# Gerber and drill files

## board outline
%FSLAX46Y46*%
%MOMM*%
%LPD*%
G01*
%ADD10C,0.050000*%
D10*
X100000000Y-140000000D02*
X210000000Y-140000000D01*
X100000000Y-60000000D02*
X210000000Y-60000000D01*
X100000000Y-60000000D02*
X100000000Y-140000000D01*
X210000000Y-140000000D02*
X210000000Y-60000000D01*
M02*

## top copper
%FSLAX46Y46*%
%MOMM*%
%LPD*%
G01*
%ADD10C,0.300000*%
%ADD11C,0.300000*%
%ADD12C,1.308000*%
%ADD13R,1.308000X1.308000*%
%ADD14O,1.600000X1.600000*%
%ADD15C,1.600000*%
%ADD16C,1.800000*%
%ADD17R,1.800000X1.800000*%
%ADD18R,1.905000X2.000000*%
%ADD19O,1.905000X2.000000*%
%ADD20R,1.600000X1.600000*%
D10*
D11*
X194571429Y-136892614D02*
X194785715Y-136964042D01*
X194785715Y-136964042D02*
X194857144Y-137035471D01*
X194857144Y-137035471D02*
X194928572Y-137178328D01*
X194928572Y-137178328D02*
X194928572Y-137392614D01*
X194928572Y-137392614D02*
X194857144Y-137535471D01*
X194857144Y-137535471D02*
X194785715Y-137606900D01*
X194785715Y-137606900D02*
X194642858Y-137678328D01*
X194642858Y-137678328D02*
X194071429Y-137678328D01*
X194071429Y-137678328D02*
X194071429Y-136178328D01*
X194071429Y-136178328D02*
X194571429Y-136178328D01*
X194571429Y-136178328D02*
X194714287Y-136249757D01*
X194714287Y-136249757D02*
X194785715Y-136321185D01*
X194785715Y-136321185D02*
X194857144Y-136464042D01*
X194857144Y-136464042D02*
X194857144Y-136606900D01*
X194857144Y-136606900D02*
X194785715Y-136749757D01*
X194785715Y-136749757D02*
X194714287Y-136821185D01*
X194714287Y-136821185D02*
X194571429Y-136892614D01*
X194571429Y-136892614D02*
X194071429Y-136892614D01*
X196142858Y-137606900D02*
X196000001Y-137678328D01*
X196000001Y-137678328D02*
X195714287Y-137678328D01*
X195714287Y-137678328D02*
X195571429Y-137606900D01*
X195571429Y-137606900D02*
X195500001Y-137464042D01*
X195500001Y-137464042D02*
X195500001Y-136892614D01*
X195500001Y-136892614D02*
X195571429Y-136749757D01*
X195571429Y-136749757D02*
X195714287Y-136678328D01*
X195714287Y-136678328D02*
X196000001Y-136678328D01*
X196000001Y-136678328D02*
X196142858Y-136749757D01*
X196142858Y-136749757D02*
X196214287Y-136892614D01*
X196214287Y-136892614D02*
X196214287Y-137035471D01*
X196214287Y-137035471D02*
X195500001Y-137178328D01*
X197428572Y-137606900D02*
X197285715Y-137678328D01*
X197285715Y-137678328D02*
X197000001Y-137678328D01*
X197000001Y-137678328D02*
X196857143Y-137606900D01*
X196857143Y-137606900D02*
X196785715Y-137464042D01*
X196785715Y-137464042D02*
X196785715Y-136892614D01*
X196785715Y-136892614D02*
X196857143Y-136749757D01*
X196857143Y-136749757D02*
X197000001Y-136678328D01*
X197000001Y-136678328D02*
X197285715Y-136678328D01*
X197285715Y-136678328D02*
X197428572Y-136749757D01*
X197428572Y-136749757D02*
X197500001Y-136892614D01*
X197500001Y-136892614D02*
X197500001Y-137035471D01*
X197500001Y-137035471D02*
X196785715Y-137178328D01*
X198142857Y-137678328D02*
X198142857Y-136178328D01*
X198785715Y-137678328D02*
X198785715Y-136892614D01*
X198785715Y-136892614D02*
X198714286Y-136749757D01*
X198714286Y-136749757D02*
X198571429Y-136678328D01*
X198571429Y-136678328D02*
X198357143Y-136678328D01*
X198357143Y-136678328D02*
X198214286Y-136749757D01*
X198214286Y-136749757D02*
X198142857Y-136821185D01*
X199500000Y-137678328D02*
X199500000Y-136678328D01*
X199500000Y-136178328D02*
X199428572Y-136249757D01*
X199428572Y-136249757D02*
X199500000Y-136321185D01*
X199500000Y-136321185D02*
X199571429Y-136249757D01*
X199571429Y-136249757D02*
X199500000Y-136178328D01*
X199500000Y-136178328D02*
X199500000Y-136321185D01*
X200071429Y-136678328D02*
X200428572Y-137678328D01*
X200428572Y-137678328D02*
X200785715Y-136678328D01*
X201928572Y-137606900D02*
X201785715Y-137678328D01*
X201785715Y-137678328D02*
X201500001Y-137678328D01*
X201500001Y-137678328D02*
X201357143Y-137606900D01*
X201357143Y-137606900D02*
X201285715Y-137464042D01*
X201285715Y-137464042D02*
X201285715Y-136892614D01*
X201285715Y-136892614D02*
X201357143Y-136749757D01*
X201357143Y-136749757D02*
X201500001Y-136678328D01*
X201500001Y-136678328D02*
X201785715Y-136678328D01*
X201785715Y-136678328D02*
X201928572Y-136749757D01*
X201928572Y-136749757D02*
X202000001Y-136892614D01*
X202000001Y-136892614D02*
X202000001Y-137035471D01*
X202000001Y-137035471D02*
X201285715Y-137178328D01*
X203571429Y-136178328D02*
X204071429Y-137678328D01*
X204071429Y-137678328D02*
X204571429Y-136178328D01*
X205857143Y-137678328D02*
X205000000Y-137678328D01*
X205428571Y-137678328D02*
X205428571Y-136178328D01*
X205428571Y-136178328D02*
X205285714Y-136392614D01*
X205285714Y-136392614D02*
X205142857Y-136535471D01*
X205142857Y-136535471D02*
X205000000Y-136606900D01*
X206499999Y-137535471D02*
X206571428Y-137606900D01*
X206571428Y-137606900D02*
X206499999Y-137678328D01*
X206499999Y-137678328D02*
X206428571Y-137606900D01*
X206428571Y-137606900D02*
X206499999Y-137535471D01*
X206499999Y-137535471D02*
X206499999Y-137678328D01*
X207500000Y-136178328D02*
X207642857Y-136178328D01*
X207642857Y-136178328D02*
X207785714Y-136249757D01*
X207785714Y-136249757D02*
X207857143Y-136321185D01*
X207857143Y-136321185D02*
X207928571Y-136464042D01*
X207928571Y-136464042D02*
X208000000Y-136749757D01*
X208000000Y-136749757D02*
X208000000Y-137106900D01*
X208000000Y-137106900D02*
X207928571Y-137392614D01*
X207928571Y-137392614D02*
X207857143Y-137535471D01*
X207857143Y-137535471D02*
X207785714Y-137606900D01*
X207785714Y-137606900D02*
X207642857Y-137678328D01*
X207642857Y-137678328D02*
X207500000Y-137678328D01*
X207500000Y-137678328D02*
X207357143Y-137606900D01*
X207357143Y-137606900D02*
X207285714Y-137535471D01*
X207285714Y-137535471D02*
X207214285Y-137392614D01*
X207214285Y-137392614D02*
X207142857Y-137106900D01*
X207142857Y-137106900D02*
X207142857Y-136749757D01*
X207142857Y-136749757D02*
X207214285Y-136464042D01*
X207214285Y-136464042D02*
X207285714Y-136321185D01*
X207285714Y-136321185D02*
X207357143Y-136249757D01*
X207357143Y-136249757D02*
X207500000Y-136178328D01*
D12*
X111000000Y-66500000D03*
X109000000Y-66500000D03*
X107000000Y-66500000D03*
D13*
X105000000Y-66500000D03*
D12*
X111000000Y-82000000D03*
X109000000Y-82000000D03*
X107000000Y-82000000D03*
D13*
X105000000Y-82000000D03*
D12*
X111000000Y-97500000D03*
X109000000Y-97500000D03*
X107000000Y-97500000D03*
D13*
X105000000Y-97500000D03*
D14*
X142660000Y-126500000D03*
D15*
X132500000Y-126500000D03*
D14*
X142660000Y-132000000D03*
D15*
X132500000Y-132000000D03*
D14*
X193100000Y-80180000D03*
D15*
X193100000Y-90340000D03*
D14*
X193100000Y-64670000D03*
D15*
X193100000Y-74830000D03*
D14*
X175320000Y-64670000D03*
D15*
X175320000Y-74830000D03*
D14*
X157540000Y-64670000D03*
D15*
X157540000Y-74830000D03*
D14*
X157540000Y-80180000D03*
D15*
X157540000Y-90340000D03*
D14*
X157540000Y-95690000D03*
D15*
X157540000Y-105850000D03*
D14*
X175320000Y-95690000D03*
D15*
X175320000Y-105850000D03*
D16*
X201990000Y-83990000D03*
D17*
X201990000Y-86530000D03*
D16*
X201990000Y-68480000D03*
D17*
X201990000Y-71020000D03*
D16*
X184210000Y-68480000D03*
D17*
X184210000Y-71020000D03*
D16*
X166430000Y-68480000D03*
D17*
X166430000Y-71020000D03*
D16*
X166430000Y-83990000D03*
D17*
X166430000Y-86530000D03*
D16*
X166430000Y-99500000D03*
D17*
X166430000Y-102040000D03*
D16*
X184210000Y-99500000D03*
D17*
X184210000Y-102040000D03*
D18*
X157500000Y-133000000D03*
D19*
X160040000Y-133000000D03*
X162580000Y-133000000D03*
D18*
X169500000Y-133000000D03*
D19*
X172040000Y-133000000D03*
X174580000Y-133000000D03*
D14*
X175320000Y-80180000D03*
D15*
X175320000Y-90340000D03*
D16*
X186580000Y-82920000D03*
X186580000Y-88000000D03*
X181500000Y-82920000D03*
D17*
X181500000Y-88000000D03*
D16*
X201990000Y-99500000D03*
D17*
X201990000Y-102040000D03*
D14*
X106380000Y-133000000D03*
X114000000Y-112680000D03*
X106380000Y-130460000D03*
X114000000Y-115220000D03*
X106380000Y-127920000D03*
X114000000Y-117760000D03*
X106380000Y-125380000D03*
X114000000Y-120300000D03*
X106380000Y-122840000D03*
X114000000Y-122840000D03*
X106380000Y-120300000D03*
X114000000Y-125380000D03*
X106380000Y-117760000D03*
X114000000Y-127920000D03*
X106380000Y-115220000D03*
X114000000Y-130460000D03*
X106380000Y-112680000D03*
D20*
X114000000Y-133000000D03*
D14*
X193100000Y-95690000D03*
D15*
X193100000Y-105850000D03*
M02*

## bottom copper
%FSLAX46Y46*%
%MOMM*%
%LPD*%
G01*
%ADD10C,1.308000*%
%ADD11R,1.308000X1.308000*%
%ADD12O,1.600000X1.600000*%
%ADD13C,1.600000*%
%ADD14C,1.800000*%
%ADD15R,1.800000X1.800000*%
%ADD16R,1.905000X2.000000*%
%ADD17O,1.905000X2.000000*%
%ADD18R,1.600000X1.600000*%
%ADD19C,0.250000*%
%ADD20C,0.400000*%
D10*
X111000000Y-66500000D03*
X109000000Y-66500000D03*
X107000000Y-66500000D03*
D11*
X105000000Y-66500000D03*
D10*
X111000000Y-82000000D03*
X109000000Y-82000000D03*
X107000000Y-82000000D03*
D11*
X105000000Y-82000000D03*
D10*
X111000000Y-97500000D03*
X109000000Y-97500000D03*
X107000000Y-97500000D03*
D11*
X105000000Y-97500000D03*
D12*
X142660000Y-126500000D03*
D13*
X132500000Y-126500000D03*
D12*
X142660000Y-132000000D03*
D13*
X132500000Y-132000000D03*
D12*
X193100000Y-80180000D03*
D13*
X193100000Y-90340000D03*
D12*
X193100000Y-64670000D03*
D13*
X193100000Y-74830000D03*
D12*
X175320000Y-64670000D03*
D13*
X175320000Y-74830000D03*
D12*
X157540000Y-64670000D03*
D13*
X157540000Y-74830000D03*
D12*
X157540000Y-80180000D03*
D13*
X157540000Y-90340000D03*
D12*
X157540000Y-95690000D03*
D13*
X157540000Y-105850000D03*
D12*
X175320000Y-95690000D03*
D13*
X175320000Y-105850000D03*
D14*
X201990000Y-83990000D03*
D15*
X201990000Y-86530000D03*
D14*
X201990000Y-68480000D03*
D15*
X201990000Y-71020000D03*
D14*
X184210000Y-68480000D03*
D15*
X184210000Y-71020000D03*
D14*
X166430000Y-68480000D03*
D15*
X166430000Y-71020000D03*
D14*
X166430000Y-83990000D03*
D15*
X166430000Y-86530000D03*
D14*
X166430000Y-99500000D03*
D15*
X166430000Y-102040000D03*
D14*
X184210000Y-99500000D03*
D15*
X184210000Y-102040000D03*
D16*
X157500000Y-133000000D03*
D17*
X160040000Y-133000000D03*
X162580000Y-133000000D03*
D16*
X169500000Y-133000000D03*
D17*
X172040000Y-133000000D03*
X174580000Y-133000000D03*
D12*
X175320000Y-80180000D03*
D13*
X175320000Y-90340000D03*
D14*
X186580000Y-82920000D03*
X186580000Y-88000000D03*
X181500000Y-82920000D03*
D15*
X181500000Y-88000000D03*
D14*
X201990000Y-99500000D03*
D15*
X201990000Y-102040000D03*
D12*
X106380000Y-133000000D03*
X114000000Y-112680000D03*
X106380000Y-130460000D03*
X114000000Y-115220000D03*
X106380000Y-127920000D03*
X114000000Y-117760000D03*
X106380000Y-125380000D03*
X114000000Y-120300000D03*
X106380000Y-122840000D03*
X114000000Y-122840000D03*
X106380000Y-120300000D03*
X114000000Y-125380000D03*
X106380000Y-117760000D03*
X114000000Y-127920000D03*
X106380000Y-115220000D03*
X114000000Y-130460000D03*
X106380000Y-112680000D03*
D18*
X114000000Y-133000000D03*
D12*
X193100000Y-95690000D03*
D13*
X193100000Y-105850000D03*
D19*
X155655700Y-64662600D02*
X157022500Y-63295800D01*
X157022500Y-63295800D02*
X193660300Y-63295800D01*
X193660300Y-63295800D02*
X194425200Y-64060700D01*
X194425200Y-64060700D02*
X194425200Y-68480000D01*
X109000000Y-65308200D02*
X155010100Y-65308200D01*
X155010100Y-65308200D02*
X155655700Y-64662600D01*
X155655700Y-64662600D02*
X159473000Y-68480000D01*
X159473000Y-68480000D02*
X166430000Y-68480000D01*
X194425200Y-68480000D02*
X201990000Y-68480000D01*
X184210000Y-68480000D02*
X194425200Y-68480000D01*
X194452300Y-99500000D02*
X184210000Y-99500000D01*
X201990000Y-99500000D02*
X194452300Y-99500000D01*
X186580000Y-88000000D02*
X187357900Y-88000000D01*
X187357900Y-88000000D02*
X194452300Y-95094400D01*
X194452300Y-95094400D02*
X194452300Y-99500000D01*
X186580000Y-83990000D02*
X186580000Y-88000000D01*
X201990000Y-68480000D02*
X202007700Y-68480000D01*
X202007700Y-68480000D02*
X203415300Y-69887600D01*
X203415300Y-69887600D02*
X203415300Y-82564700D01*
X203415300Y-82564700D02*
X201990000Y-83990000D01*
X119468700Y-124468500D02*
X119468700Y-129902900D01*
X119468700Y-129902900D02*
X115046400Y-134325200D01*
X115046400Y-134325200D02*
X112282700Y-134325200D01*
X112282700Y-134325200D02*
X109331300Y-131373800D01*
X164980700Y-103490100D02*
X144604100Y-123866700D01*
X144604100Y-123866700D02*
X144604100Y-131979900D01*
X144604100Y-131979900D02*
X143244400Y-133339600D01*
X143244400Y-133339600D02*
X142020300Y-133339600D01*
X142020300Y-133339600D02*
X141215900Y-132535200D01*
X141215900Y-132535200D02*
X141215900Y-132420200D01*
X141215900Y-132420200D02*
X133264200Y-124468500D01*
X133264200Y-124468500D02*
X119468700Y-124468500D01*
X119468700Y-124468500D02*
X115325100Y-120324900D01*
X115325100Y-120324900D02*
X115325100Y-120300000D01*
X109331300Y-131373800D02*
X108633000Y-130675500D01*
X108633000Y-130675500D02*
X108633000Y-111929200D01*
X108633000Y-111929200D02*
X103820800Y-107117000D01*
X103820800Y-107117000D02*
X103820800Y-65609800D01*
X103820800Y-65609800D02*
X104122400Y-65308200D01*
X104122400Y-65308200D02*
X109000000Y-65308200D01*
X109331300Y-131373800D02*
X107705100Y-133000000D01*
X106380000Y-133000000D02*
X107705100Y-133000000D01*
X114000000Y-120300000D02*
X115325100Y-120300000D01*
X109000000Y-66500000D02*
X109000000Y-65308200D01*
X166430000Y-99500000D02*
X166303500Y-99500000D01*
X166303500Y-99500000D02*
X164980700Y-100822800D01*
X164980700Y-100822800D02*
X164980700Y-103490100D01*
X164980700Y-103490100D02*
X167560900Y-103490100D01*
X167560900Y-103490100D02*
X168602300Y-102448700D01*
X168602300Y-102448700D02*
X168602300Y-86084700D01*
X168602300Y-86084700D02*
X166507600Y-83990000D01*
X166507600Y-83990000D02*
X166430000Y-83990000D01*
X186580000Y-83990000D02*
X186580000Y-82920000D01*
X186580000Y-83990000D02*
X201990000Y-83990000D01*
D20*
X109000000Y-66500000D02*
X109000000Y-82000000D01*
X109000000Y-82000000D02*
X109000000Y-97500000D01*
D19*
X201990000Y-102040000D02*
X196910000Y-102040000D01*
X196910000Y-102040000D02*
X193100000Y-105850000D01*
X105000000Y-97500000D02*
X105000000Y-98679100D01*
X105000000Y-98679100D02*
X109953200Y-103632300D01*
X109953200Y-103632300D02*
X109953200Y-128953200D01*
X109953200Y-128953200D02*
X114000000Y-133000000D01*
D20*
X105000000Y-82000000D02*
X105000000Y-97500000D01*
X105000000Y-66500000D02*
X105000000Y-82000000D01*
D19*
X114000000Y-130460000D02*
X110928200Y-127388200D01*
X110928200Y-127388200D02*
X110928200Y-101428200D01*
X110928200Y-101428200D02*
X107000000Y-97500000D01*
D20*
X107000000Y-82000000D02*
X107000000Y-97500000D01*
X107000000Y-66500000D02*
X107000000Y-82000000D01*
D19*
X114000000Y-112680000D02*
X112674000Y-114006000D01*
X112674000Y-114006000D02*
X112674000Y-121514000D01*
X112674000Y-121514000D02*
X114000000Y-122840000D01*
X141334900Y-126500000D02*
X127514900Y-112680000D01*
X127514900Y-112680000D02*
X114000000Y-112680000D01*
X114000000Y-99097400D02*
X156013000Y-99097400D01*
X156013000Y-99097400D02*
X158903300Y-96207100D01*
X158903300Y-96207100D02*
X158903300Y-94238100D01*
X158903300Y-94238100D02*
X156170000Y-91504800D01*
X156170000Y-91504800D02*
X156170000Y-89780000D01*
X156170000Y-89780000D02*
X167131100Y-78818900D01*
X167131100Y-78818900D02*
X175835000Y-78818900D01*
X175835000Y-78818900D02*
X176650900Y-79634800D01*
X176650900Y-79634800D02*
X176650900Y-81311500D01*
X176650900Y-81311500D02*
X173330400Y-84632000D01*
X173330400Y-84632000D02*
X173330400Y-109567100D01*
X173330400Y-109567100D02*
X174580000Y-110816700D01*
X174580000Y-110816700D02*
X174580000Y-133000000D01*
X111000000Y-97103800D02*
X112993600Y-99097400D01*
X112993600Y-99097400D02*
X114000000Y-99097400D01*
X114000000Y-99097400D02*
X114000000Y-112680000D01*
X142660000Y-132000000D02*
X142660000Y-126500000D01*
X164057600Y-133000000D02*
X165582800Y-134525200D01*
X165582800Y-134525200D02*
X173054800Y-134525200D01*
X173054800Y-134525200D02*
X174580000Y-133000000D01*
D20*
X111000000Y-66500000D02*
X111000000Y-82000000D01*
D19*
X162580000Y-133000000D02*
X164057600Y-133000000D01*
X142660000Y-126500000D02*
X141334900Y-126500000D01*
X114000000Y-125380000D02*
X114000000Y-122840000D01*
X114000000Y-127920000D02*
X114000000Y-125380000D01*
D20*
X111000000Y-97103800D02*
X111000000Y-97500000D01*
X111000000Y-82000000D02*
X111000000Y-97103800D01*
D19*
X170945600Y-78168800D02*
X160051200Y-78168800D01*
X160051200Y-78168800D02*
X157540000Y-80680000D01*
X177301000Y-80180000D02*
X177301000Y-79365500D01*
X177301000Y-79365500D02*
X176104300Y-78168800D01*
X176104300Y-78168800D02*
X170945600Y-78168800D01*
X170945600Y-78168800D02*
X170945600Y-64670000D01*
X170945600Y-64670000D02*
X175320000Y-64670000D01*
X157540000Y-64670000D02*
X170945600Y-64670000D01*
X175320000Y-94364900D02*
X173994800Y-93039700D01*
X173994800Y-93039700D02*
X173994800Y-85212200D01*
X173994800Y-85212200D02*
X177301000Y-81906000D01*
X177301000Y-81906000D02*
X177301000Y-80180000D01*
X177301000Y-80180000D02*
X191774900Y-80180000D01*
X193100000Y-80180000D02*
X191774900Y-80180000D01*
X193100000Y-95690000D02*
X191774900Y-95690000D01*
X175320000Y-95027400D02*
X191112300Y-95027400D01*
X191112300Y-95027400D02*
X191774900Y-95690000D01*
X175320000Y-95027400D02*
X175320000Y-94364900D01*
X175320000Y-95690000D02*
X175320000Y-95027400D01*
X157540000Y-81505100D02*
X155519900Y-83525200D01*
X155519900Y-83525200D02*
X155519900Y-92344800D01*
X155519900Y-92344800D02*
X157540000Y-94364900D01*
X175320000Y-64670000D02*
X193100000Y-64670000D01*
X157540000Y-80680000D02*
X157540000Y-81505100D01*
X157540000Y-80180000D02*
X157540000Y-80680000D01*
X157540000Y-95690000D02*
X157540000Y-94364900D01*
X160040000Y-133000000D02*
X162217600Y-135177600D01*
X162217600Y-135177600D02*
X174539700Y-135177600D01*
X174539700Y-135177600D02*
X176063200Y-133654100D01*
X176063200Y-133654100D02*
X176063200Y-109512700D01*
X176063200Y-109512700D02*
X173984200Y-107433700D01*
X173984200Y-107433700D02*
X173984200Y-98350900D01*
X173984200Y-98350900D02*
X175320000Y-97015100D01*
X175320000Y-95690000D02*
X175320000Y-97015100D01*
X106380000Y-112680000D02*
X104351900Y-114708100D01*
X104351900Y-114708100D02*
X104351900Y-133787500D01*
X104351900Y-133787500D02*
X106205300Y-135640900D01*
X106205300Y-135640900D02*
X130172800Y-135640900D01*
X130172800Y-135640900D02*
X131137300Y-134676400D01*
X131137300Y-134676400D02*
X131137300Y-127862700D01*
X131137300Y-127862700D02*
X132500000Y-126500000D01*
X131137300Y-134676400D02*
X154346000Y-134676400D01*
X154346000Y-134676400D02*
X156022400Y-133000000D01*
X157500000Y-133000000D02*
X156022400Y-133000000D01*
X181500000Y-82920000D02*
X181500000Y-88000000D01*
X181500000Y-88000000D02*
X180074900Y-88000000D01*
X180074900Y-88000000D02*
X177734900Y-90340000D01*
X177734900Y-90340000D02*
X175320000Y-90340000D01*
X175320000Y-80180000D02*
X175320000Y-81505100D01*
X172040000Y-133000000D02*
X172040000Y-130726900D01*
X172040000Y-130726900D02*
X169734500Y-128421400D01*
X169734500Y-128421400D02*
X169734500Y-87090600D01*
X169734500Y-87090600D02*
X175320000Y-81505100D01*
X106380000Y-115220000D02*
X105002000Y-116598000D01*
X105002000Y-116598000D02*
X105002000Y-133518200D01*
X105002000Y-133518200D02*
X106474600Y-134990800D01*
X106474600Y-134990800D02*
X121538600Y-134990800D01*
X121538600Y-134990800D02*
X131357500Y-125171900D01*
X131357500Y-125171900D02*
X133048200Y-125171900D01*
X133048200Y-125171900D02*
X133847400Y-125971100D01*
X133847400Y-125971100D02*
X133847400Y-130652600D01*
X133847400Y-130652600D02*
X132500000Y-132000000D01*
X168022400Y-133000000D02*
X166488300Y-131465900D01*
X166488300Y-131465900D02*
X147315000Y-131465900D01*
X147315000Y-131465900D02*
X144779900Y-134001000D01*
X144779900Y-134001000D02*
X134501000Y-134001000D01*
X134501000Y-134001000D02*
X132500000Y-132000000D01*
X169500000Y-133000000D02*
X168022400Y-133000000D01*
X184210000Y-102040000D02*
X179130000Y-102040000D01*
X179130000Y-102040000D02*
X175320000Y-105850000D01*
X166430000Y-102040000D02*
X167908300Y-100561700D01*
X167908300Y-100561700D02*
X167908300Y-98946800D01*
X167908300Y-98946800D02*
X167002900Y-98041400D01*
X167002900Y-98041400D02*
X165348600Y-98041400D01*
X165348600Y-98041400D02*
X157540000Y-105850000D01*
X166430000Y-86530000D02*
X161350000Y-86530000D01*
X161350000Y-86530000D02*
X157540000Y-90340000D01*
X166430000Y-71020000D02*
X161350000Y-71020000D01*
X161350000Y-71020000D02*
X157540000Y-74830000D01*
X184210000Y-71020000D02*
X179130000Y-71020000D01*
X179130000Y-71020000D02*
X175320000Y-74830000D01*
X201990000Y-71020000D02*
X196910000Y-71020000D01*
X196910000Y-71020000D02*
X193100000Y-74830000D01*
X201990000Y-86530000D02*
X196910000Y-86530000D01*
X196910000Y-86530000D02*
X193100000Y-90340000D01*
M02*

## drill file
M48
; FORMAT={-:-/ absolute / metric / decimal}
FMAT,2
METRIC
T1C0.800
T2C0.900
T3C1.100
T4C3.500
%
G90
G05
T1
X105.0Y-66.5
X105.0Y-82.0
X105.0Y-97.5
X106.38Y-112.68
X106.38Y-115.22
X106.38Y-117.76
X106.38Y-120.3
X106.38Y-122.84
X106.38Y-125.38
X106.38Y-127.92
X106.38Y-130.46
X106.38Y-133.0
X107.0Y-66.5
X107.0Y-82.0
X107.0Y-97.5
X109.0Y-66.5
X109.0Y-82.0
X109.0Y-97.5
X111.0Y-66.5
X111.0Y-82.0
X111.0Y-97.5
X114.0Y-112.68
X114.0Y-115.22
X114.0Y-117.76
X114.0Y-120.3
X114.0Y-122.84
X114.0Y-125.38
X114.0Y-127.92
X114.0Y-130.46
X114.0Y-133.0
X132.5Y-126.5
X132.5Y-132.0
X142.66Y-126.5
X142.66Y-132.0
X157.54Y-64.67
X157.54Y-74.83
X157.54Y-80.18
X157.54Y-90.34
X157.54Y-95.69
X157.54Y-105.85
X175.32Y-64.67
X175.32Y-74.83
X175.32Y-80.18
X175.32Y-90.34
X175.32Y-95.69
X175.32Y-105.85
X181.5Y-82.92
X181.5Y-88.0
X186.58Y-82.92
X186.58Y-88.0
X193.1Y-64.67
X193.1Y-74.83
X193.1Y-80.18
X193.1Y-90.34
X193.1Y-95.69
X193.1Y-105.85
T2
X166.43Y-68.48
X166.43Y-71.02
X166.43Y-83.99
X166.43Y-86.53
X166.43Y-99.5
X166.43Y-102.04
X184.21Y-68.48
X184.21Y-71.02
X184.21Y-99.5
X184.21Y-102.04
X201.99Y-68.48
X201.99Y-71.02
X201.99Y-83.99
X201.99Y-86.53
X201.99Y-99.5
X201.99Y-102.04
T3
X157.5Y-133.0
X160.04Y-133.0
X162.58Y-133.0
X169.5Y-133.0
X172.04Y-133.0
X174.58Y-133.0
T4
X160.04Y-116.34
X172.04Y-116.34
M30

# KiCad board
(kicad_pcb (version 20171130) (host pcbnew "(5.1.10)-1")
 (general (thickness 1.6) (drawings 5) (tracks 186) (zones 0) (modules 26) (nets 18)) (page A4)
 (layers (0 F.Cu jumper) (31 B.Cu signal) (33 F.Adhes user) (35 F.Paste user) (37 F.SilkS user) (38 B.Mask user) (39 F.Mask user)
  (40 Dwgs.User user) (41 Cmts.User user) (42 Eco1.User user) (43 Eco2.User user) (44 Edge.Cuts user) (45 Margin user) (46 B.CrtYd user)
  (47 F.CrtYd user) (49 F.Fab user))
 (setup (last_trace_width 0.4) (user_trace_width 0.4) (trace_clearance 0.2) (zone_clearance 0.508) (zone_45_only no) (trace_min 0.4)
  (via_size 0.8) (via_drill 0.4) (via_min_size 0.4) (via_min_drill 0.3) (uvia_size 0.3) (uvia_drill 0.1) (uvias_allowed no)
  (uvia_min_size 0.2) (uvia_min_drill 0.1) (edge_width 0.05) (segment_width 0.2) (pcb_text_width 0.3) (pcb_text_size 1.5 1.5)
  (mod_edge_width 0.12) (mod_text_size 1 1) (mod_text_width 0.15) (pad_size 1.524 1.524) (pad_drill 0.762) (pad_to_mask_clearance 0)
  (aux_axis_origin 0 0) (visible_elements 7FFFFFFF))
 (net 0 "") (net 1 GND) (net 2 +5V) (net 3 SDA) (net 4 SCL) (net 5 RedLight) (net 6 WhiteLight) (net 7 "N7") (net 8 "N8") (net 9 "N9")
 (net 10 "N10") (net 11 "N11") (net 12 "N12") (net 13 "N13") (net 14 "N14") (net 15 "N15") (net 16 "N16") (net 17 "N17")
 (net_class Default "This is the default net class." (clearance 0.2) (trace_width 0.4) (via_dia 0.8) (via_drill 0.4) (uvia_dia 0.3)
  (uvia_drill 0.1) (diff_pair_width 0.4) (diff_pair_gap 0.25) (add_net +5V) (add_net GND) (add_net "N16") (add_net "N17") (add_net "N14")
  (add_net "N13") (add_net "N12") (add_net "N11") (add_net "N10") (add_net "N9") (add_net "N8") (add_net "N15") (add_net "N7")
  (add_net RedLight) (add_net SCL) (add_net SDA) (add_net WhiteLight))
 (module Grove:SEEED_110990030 (layer F.Cu) (at 108 66.5)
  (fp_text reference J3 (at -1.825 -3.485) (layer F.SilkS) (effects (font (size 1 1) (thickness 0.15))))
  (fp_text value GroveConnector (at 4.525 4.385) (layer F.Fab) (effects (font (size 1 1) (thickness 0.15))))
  (pad 4 thru_hole circle (at 3 0) (size 1.308 1.308) (drill 0.8) (layers *.Cu *.Mask) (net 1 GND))
  (pad 3 thru_hole circle (at 1 0) (size 1.308 1.308) (drill 0.8) (layers *.Cu *.Mask) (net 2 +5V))
  (pad 2 thru_hole circle (at -1 0) (size 1.308 1.308) (drill 0.8) (layers *.Cu *.Mask) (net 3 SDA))
  (pad 1 thru_hole rect (at -3 0) (size 1.308 1.308) (drill 0.8) (layers *.Cu *.Mask) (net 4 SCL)))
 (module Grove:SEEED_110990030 (layer F.Cu) (at 108 82)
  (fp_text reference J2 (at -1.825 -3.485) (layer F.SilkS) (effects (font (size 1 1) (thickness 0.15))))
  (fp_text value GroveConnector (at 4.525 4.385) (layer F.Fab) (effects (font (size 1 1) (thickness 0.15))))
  (pad 4 thru_hole circle (at 3 0) (size 1.308 1.308) (drill 0.8) (layers *.Cu *.Mask) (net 1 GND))
  (pad 3 thru_hole circle (at 1 0) (size 1.308 1.308) (drill 0.8) (layers *.Cu *.Mask) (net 2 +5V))
  (pad 2 thru_hole circle (at -1 0) (size 1.308 1.308) (drill 0.8) (layers *.Cu *.Mask) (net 3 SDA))
  (pad 1 thru_hole rect (at -3 0) (size 1.308 1.308) (drill 0.8) (layers *.Cu *.Mask) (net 4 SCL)))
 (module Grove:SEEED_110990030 (layer F.Cu) (at 108 97.5)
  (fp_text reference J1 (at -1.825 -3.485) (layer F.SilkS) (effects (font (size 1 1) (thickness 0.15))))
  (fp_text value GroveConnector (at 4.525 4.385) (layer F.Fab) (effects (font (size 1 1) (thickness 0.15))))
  (pad 4 thru_hole circle (at 3 0) (size 1.308 1.308) (drill 0.8) (layers *.Cu *.Mask) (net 1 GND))
  (pad 3 thru_hole circle (at 1 0) (size 1.308 1.308) (drill 0.8) (layers *.Cu *.Mask) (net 2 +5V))
  (pad 2 thru_hole circle (at -1 0) (size 1.308 1.308) (drill 0.8) (layers *.Cu *.Mask) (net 3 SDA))
  (pad 1 thru_hole rect (at -3 0) (size 1.308 1.308) (drill 0.8) (layers *.Cu *.Mask) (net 4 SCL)))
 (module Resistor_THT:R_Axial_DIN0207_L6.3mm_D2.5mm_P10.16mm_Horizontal (layer F.Cu) (at 132.5 126.5)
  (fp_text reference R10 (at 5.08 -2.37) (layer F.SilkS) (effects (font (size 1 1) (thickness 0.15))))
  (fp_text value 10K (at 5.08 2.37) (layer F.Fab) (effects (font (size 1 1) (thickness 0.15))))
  (pad 2 thru_hole oval (at 10.16 0) (size 1.6 1.6) (drill 0.8) (layers *.Cu *.Mask) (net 1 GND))
  (pad 1 thru_hole circle (at 0 0) (size 1.6 1.6) (drill 0.8) (layers *.Cu *.Mask) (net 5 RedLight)))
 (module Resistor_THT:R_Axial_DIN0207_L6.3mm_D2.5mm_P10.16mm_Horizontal (layer F.Cu) (at 132.5 132)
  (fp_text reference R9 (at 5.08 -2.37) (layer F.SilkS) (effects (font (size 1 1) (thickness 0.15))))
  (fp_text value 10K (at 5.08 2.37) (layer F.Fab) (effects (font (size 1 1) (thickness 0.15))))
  (pad 2 thru_hole oval (at 10.16 0) (size 1.6 1.6) (drill 0.8) (layers *.Cu *.Mask) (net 1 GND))
  (pad 1 thru_hole circle (at 0 0) (size 1.6 1.6) (drill 0.8) (layers *.Cu *.Mask) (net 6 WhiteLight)))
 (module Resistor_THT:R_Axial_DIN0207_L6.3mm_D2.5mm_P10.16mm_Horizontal (layer F.Cu) (at 193.1 90.34 90)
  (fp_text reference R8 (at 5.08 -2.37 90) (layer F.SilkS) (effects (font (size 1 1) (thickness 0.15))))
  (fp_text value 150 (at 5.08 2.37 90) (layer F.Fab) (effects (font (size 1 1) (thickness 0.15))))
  (pad 2 thru_hole oval (at 10.16 0 90) (size 1.6 1.6) (drill 0.8) (layers *.Cu *.Mask) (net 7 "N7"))
  (pad 1 thru_hole circle (at 0 0 90) (size 1.6 1.6) (drill 0.8) (layers *.Cu *.Mask) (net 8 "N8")))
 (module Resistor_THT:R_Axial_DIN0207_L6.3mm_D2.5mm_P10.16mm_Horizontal (layer F.Cu) (at 193.1 74.83 90)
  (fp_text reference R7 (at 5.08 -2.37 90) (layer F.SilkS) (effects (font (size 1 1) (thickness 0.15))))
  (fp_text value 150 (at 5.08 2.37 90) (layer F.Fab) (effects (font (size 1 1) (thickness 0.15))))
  (pad 2 thru_hole oval (at 10.16 0 90) (size 1.6 1.6) (drill 0.8) (layers *.Cu *.Mask) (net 7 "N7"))
  (pad 1 thru_hole circle (at 0 0 90) (size 1.6 1.6) (drill 0.8) (layers *.Cu *.Mask) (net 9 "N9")))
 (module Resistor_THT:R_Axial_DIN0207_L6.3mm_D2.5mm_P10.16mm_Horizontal (layer F.Cu) (at 175.32 74.83 90)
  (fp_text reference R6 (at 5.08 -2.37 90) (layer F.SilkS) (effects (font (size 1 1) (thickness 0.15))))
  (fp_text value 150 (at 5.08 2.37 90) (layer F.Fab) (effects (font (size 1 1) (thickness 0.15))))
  (pad 2 thru_hole oval (at 10.16 0 90) (size 1.6 1.6) (drill 0.8) (layers *.Cu *.Mask) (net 7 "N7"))
  (pad 1 thru_hole circle (at 0 0 90) (size 1.6 1.6) (drill 0.8) (layers *.Cu *.Mask) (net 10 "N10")))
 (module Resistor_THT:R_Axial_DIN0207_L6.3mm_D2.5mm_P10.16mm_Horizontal (layer F.Cu) (at 157.54 74.83 90)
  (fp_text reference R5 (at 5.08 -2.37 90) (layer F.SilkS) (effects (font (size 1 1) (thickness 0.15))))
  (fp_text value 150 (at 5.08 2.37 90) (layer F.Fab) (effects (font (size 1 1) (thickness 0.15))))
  (pad 2 thru_hole oval (at 10.16 0 90) (size 1.6 1.6) (drill 0.8) (layers *.Cu *.Mask) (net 7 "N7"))
  (pad 1 thru_hole circle (at 0 0 90) (size 1.6 1.6) (drill 0.8) (layers *.Cu *.Mask) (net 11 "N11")))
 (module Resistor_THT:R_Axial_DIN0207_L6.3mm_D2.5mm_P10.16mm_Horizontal (layer F.Cu) (at 157.54 90.34 90)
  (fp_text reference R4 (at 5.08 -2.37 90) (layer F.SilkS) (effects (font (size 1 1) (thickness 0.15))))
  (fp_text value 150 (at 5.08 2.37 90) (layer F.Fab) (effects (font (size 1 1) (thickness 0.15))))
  (pad 2 thru_hole oval (at 10.16 0 90) (size 1.6 1.6) (drill 0.8) (layers *.Cu *.Mask) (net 7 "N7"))
  (pad 1 thru_hole circle (at 0 0 90) (size 1.6 1.6) (drill 0.8) (layers *.Cu *.Mask) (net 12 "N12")))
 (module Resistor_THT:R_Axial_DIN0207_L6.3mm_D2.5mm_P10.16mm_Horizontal (layer F.Cu) (at 157.54 105.85 90)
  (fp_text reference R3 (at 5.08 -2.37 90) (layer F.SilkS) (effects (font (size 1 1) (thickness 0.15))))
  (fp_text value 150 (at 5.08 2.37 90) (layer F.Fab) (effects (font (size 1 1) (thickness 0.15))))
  (pad 2 thru_hole oval (at 10.16 0 90) (size 1.6 1.6) (drill 0.8) (layers *.Cu *.Mask) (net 7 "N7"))
  (pad 1 thru_hole circle (at 0 0 90) (size 1.6 1.6) (drill 0.8) (layers *.Cu *.Mask) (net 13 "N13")))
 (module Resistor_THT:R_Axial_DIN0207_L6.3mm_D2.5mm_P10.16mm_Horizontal (layer F.Cu) (at 175.32 105.85 90)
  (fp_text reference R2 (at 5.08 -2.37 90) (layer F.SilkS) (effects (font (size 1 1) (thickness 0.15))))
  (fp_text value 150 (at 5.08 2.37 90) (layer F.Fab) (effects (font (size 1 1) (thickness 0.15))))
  (pad 2 thru_hole oval (at 10.16 0 90) (size 1.6 1.6) (drill 0.8) (layers *.Cu *.Mask) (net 7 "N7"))
  (pad 1 thru_hole circle (at 0 0 90) (size 1.6 1.6) (drill 0.8) (layers *.Cu *.Mask) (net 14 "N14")))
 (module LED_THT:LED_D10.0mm (layer F.Cu) (at 201.99 86.53 90)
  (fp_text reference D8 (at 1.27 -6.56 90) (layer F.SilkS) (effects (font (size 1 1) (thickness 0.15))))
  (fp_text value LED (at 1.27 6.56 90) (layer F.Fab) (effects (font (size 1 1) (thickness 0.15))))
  (pad 2 thru_hole circle (at 2.54 0 90) (size 1.8 1.8) (drill 0.9) (layers *.Cu *.Mask) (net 2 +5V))
  (pad 1 thru_hole rect (at 0 0 90) (size 1.8 1.8) (drill 0.9) (layers *.Cu *.Mask) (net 8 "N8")))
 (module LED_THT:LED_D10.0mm (layer F.Cu) (at 201.99 71.02 90)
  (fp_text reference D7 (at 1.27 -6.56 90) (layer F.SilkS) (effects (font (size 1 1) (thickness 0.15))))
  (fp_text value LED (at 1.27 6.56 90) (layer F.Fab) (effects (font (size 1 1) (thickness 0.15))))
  (pad 2 thru_hole circle (at 2.54 0 90) (size 1.8 1.8) (drill 0.9) (layers *.Cu *.Mask) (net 2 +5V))
  (pad 1 thru_hole rect (at 0 0 90) (size 1.8 1.8) (drill 0.9) (layers *.Cu *.Mask) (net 9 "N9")))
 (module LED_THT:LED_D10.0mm (layer F.Cu) (at 184.21 71.02 90)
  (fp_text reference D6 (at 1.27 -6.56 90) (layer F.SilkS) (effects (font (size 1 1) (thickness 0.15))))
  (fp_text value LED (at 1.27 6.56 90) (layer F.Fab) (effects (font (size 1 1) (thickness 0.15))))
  (pad 2 thru_hole circle (at 2.54 0 90) (size 1.8 1.8) (drill 0.9) (layers *.Cu *.Mask) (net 2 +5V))
  (pad 1 thru_hole rect (at 0 0 90) (size 1.8 1.8) (drill 0.9) (layers *.Cu *.Mask) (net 10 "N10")))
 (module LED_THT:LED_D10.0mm (layer F.Cu) (at 166.43 71.02 90)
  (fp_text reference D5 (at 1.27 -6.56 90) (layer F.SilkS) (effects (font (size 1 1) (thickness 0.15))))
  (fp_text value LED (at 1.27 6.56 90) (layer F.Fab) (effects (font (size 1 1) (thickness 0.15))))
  (pad 2 thru_hole circle (at 2.54 0 90) (size 1.8 1.8) (drill 0.9) (layers *.Cu *.Mask) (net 2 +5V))
  (pad 1 thru_hole rect (at 0 0 90) (size 1.8 1.8) (drill 0.9) (layers *.Cu *.Mask) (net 11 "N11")))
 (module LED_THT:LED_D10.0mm (layer F.Cu) (at 166.43 86.53 90)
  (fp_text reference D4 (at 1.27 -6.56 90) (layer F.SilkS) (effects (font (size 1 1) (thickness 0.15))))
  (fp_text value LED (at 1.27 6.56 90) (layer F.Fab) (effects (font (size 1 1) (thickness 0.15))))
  (pad 2 thru_hole circle (at 2.54 0 90) (size 1.8 1.8) (drill 0.9) (layers *.Cu *.Mask) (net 2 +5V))
  (pad 1 thru_hole rect (at 0 0 90) (size 1.8 1.8) (drill 0.9) (layers *.Cu *.Mask) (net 12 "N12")))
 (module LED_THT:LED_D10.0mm (layer F.Cu) (at 166.43 102.04 90)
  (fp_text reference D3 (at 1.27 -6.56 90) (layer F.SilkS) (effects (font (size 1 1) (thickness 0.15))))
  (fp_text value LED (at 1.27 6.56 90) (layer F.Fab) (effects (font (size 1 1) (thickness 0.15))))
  (pad 2 thru_hole circle (at 2.54 0 90) (size 1.8 1.8) (drill 0.9) (layers *.Cu *.Mask) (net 2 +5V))
  (pad 1 thru_hole rect (at 0 0 90) (size 1.8 1.8) (drill 0.9) (layers *.Cu *.Mask) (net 13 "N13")))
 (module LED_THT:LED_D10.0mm (layer F.Cu) (at 184.21 102.04 90)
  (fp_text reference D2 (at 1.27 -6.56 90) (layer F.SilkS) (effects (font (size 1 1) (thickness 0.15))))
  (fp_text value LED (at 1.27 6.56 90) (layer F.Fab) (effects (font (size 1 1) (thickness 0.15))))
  (pad 2 thru_hole circle (at 2.54 0 90) (size 1.8 1.8) (drill 0.9) (layers *.Cu *.Mask) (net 2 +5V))
  (pad 1 thru_hole rect (at 0 0 90) (size 1.8 1.8) (drill 0.9) (layers *.Cu *.Mask) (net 14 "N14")))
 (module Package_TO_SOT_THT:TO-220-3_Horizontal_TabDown (layer F.Cu) (at 157.5 133)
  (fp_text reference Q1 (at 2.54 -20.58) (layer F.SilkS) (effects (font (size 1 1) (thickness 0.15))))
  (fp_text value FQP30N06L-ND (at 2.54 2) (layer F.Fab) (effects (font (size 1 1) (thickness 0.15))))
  (pad "" np_thru_hole oval (at 2.54 -16.66) (size 3.5 3.5) (drill 3.5) (layers *.Cu *.Mask))
  (pad 1 thru_hole rect (at 0 0) (size 1.905 2) (drill 1.1) (layers *.Cu *.Mask) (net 5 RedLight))
  (pad 2 thru_hole oval (at 2.54 0) (size 1.905 2) (drill 1.1) (layers *.Cu *.Mask) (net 7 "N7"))
  (pad 3 thru_hole oval (at 5.08 0) (size 1.905 2) (drill 1.1) (layers *.Cu *.Mask) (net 1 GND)))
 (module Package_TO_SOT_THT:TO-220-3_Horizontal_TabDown (layer F.Cu) (at 169.5 133)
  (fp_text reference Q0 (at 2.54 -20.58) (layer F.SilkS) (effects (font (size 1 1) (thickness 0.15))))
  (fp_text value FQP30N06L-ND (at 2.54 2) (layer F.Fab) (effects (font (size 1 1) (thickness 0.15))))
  (pad "" np_thru_hole oval (at 2.54 -16.66) (size 3.5 3.5) (drill 3.5) (layers *.Cu *.Mask))
  (pad 1 thru_hole rect (at 0 0) (size 1.905 2) (drill 1.1) (layers *.Cu *.Mask) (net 6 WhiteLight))
  (pad 2 thru_hole oval (at 2.54 0) (size 1.905 2) (drill 1.1) (layers *.Cu *.Mask) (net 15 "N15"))
  (pad 3 thru_hole oval (at 5.08 0) (size 1.905 2) (drill 1.1) (layers *.Cu *.Mask) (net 1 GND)))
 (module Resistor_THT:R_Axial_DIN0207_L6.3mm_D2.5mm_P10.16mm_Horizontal (layer F.Cu) (at 175.32 90.34 90)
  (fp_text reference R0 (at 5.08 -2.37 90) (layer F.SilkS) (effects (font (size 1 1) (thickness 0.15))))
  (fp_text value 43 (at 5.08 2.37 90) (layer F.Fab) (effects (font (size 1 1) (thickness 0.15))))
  (pad 2 thru_hole oval (at 10.16 0 90) (size 1.6 1.6) (drill 0.8) (layers *.Cu *.Mask) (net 15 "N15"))
  (pad 1 thru_hole circle (at 0 0 90) (size 1.6 1.6) (drill 0.8) (layers *.Cu *.Mask) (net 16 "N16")))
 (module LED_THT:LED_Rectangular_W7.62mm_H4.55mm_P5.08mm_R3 (layer F.Cu) (at 181.5 88 90)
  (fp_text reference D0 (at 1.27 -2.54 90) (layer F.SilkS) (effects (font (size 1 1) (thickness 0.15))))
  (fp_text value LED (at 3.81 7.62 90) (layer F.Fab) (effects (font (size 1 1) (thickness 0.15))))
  (pad 2 thru_hole circle (at 5.08 5.08 90) (size 1.8 1.8) (drill 0.8) (layers *.Cu *.Mask) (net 2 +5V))
  (pad 2 thru_hole circle (at 0 5.08 90) (size 1.8 1.8) (drill 0.8) (layers *.Cu *.Mask) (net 2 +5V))
  (pad 1 thru_hole circle (at 5.08 0 90) (size 1.8 1.8) (drill 0.8) (layers *.Cu *.Mask) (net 16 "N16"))
  (pad 1 thru_hole rect (at 0 0 90) (size 1.8 1.8) (drill 0.8) (layers *.Cu *.Mask) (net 16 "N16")))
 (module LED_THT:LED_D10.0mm (layer F.Cu) (at 201.99 102.04 90)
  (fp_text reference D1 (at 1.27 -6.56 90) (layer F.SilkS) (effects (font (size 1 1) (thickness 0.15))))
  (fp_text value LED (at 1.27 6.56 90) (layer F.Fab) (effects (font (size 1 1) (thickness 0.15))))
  (pad 2 thru_hole circle (at 2.54 0 90) (size 1.8 1.8) (drill 0.9) (layers *.Cu *.Mask) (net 2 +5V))
  (pad 1 thru_hole rect (at 0 0 90) (size 1.8 1.8) (drill 0.9) (layers *.Cu *.Mask) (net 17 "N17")))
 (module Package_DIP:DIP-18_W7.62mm (layer F.Cu) (at 114 133 180)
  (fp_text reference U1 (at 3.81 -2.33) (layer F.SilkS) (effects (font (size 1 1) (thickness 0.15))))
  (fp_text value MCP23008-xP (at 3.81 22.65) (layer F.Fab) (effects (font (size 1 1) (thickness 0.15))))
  (pad 18 thru_hole oval (at 7.62 0 180) (size 1.6 1.6) (drill 0.8) (layers *.Cu *.Mask) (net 2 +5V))
  (pad 9 thru_hole oval (at 0 20.32 180) (size 1.6 1.6) (drill 0.8) (layers *.Cu *.Mask) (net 1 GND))
  (pad 17 thru_hole oval (at 7.62 2.54 180) (size 1.6 1.6) (drill 0.8) (layers *.Cu *.Mask))
  (pad 8 thru_hole oval (at 0 17.78 180) (size 1.6 1.6) (drill 0.8) (layers *.Cu *.Mask))
  (pad 16 thru_hole oval (at 7.62 5.08 180) (size 1.6 1.6) (drill 0.8) (layers *.Cu *.Mask))
  (pad 7 thru_hole oval (at 0 15.24 180) (size 1.6 1.6) (drill 0.8) (layers *.Cu *.Mask))
  (pad 15 thru_hole oval (at 7.62 7.62 180) (size 1.6 1.6) (drill 0.8) (layers *.Cu *.Mask))
  (pad 6 thru_hole oval (at 0 12.7 180) (size 1.6 1.6) (drill 0.8) (layers *.Cu *.Mask) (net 2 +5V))
  (pad 14 thru_hole oval (at 7.62 10.16 180) (size 1.6 1.6) (drill 0.8) (layers *.Cu *.Mask))
  (pad 5 thru_hole oval (at 0 10.16 180) (size 1.6 1.6) (drill 0.8) (layers *.Cu *.Mask) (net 1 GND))
  (pad 13 thru_hole oval (at 7.62 12.7 180) (size 1.6 1.6) (drill 0.8) (layers *.Cu *.Mask))
  (pad 4 thru_hole oval (at 0 7.62 180) (size 1.6 1.6) (drill 0.8) (layers *.Cu *.Mask) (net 1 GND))
  (pad 12 thru_hole oval (at 7.62 15.24 180) (size 1.6 1.6) (drill 0.8) (layers *.Cu *.Mask))
  (pad 3 thru_hole oval (at 0 5.08 180) (size 1.6 1.6) (drill 0.8) (layers *.Cu *.Mask) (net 1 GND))
  (pad 11 thru_hole oval (at 7.62 17.78 180) (size 1.6 1.6) (drill 0.8) (layers *.Cu *.Mask) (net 6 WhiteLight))
  (pad 2 thru_hole oval (at 0 2.54 180) (size 1.6 1.6) (drill 0.8) (layers *.Cu *.Mask) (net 3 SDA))
  (pad 10 thru_hole oval (at 7.62 20.32 180) (size 1.6 1.6) (drill 0.8) (layers *.Cu *.Mask) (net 5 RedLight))
  (pad 1 thru_hole rect (at 0 0 180) (size 1.6 1.6) (drill 0.8) (layers *.Cu *.Mask) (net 4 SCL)))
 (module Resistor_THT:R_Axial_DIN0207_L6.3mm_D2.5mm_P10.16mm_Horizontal (layer F.Cu) (at 193.1 105.85 90)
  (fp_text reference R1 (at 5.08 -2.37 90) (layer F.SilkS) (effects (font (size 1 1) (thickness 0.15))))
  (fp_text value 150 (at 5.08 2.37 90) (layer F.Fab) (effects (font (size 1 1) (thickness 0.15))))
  (pad 2 thru_hole oval (at 10.16 0 90) (size 1.6 1.6) (drill 0.8) (layers *.Cu *.Mask) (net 7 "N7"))
  (pad 1 thru_hole circle (at 0 0 90) (size 1.6 1.6) (drill 0.8) (layers *.Cu *.Mask) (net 17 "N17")))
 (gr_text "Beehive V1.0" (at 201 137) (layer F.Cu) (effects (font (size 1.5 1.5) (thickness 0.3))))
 (gr_line (start 100 140) (end 210 140) (layer Edge.Cuts) (width 0.05))
 (gr_line (start 100 60) (end 210 60) (layer Edge.Cuts) (width 0.05))
 (gr_line (start 100 60) (end 100 140) (layer Edge.Cuts) (width 0.05))
 (gr_line (start 210 140) (end 210 60) (layer Edge.Cuts) (width 0.05))
 (segment (start 155.6557 64.6626) (end 157.0225 63.2958) (width 0.25) (layer B.Cu) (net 2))
 (segment (start 157.0225 63.2958) (end 193.6603 63.2958) (width 0.25) (layer B.Cu) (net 2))
 (segment (start 193.6603 63.2958) (end 194.4252 64.0607) (width 0.25) (layer B.Cu) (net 2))
 (segment (start 194.4252 64.0607) (end 194.4252 68.48) (width 0.25) (layer B.Cu) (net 2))
 (segment (start 109 65.3082) (end 155.0101 65.3082) (width 0.25) (layer B.Cu) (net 2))
 (segment (start 155.0101 65.3082) (end 155.6557 64.6626) (width 0.25) (layer B.Cu) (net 2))
 (segment (start 155.6557 64.6626) (end 159.473 68.48) (width 0.25) (layer B.Cu) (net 2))
 (segment (start 159.473 68.48) (end 166.43 68.48) (width 0.25) (layer B.Cu) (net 2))
 (segment (start 194.4252 68.48) (end 201.99 68.48) (width 0.25) (layer B.Cu) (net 2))
 (segment (start 184.21 68.48) (end 194.4252 68.48) (width 0.25) (layer B.Cu) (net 2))
 (segment (start 194.4523 99.5) (end 184.21 99.5) (width 0.25) (layer B.Cu) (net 2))
 (segment (start 201.99 99.5) (end 194.4523 99.5) (width 0.25) (layer B.Cu) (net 2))
 (segment (start 186.58 88) (end 187.3579 88) (width 0.25) (layer B.Cu) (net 2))
 (segment (start 187.3579 88) (end 194.4523 95.0944) (width 0.25) (layer B.Cu) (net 2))
 (segment (start 194.4523 95.0944) (end 194.4523 99.5) (width 0.25) (layer B.Cu) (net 2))
 (segment (start 186.58 83.99) (end 186.58 88) (width 0.25) (layer B.Cu) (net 2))
 (segment (start 201.99 68.48) (end 202.0077 68.48) (width 0.25) (layer B.Cu) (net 2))
 (segment (start 202.0077 68.48) (end 203.4153 69.8876) (width 0.25) (layer B.Cu) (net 2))
 (segment (start 203.4153 69.8876) (end 203.4153 82.5647) (width 0.25) (layer B.Cu) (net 2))
 (segment (start 203.4153 82.5647) (end 201.99 83.99) (width 0.25) (layer B.Cu) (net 2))
 (segment (start 119.4687 124.4685) (end 119.4687 129.9029) (width 0.25) (layer B.Cu) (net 2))
 (segment (start 119.4687 129.9029) (end 115.0464 134.3252) (width 0.25) (layer B.Cu) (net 2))
 (segment (start 115.0464 134.3252) (end 112.2827 134.3252) (width 0.25) (layer B.Cu) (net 2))
 (segment (start 112.2827 134.3252) (end 109.3313 131.3738) (width 0.25) (layer B.Cu) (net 2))
 (segment (start 164.9807 103.4901) (end 144.6041 123.8667) (width 0.25) (layer B.Cu) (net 2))
 (segment (start 144.6041 123.8667) (end 144.6041 131.9799) (width 0.25) (layer B.Cu) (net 2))
 (segment (start 144.6041 131.9799) (end 143.2444 133.3396) (width 0.25) (layer B.Cu) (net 2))
 (segment (start 143.2444 133.3396) (end 142.0203 133.3396) (width 0.25) (layer B.Cu) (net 2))
 (segment (start 142.0203 133.3396) (end 141.2159 132.5352) (width 0.25) (layer B.Cu) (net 2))
 (segment (start 141.2159 132.5352) (end 141.2159 132.4202) (width 0.25) (layer B.Cu) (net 2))
 (segment (start 141.2159 132.4202) (end 133.2642 124.4685) (width 0.25) (layer B.Cu) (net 2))
 (segment (start 133.2642 124.4685) (end 119.4687 124.4685) (width 0.25) (layer B.Cu) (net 2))
 (segment (start 119.4687 124.4685) (end 115.3251 120.3249) (width 0.25) (layer B.Cu) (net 2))
 (segment (start 115.3251 120.3249) (end 115.3251 120.3) (width 0.25) (layer B.Cu) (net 2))
 (segment (start 109.3313 131.3738) (end 108.633 130.6755) (width 0.25) (layer B.Cu) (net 2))
 (segment (start 108.633 130.6755) (end 108.633 111.9292) (width 0.25) (layer B.Cu) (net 2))
 (segment (start 108.633 111.9292) (end 103.8208 107.117) (width 0.25) (layer B.Cu) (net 2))
 (segment (start 103.8208 107.117) (end 103.8208 65.6098) (width 0.25) (layer B.Cu) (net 2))
 (segment (start 103.8208 65.6098) (end 104.1224 65.3082) (width 0.25) (layer B.Cu) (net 2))
 (segment (start 104.1224 65.3082) (end 109 65.3082) (width 0.25) (layer B.Cu) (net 2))
 (segment (start 109.3313 131.3738) (end 107.7051 133) (width 0.25) (layer B.Cu) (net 2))
 (segment (start 106.38 133) (end 107.7051 133) (width 0.25) (layer B.Cu) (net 2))
 (segment (start 114 120.3) (end 115.3251 120.3) (width 0.25) (layer B.Cu) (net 2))
 (segment (start 109 66.5) (end 109 65.3082) (width 0.25) (layer B.Cu) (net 2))
 (segment (start 166.43 99.5) (end 166.3035 99.5) (width 0.25) (layer B.Cu) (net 2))
 (segment (start 166.3035 99.5) (end 164.9807 100.8228) (width 0.25) (layer B.Cu) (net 2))
 (segment (start 164.9807 100.8228) (end 164.9807 103.4901) (width 0.25) (layer B.Cu) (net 2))
 (segment (start 164.9807 103.4901) (end 167.5609 103.4901) (width 0.25) (layer B.Cu) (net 2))
 (segment (start 167.5609 103.4901) (end 168.6023 102.4487) (width 0.25) (layer B.Cu) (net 2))
 (segment (start 168.6023 102.4487) (end 168.6023 86.0847) (width 0.25) (layer B.Cu) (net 2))
 (segment (start 168.6023 86.0847) (end 166.5076 83.99) (width 0.25) (layer B.Cu) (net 2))
 (segment (start 166.5076 83.99) (end 166.43 83.99) (width 0.25) (layer B.Cu) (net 2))
 (segment (start 186.58 83.99) (end 186.58 82.92) (width 0.25) (layer B.Cu) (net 2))
 (segment (start 186.58 83.99) (end 201.99 83.99) (width 0.25) (layer B.Cu) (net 2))
 (segment (start 109 66.5) (end 109 82) (width 0.4) (layer B.Cu) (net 2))
 (segment (start 109 82) (end 109 97.5) (width 0.4) (layer B.Cu) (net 2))
 (segment (start 201.99 102.04) (end 196.91 102.04) (width 0.25) (layer B.Cu) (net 17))
 (segment (start 196.91 102.04) (end 193.1 105.85) (width 0.25) (layer B.Cu) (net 17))
 (segment (start 105 97.5) (end 105 98.6791) (width 0.25) (layer B.Cu) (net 4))
 (segment (start 105 98.6791) (end 109.9532 103.6323) (width 0.25) (layer B.Cu) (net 4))
 (segment (start 109.9532 103.6323) (end 109.9532 128.9532) (width 0.25) (layer B.Cu) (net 4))
 (segment (start 109.9532 128.9532) (end 114 133) (width 0.25) (layer B.Cu) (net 4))
 (segment (start 105 82) (end 105 97.5) (width 0.4) (layer B.Cu) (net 4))
 (segment (start 105 66.5) (end 105 82) (width 0.4) (layer B.Cu) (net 4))
 (segment (start 114 130.46) (end 110.9282 127.3882) (width 0.25) (layer B.Cu) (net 3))
 (segment (start 110.9282 127.3882) (end 110.9282 101.4282) (width 0.25) (layer B.Cu) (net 3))
 (segment (start 110.9282 101.4282) (end 107 97.5) (width 0.25) (layer B.Cu) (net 3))
 (segment (start 107 82) (end 107 97.5) (width 0.4) (layer B.Cu) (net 3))
 (segment (start 107 66.5) (end 107 82) (width 0.4) (layer B.Cu) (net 3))
 (segment (start 114 112.68) (end 112.674 114.006) (width 0.25) (layer B.Cu) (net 1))
 (segment (start 112.674 114.006) (end 112.674 121.514) (width 0.25) (layer B.Cu) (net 1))
 (segment (start 112.674 121.514) (end 114 122.84) (width 0.25) (layer B.Cu) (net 1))
 (segment (start 141.3349 126.5) (end 127.5149 112.68) (width 0.25) (layer B.Cu) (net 1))
 (segment (start 127.5149 112.68) (end 114 112.68) (width 0.25) (layer B.Cu) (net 1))
 (segment (start 114 99.0974) (end 156.013 99.0974) (width 0.25) (layer B.Cu) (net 1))
 (segment (start 156.013 99.0974) (end 158.9033 96.2071) (width 0.25) (layer B.Cu) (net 1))
 (segment (start 158.9033 96.2071) (end 158.9033 94.2381) (width 0.25) (layer B.Cu) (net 1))
 (segment (start 158.9033 94.2381) (end 156.17 91.5048) (width 0.25) (layer B.Cu) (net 1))
 (segment (start 156.17 91.5048) (end 156.17 89.78) (width 0.25) (layer B.Cu) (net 1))
 (segment (start 156.17 89.78) (end 167.1311 78.8189) (width 0.25) (layer B.Cu) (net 1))
 (segment (start 167.1311 78.8189) (end 175.835 78.8189) (width 0.25) (layer B.Cu) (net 1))
 (segment (start 175.835 78.8189) (end 176.6509 79.6348) (width 0.25) (layer B.Cu) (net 1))
 (segment (start 176.6509 79.6348) (end 176.6509 81.3115) (width 0.25) (layer B.Cu) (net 1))
 (segment (start 176.6509 81.3115) (end 173.3304 84.632) (width 0.25) (layer B.Cu) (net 1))
 (segment (start 173.3304 84.632) (end 173.3304 109.5671) (width 0.25) (layer B.Cu) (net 1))
 (segment (start 173.3304 109.5671) (end 174.58 110.8167) (width 0.25) (layer B.Cu) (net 1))
 (segment (start 174.58 110.8167) (end 174.58 133) (width 0.25) (layer B.Cu) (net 1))
 (segment (start 111 97.1038) (end 112.9936 99.0974) (width 0.25) (layer B.Cu) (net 1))
 (segment (start 112.9936 99.0974) (end 114 99.0974) (width 0.25) (layer B.Cu) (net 1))
 (segment (start 114 99.0974) (end 114 112.68) (width 0.25) (layer B.Cu) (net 1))
 (segment (start 142.66 132) (end 142.66 126.5) (width 0.25) (layer B.Cu) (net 1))
 (segment (start 164.0576 133) (end 165.5828 134.5252) (width 0.25) (layer B.Cu) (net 1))
 (segment (start 165.5828 134.5252) (end 173.0548 134.5252) (width 0.25) (layer B.Cu) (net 1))
 (segment (start 173.0548 134.5252) (end 174.58 133) (width 0.25) (layer B.Cu) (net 1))
 (segment (start 111 66.5) (end 111 82) (width 0.4) (layer B.Cu) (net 1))
 (segment (start 162.58 133) (end 164.0576 133) (width 0.25) (layer B.Cu) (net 1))
 (segment (start 142.66 126.5) (end 141.3349 126.5) (width 0.25) (layer B.Cu) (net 1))
 (segment (start 114 125.38) (end 114 122.84) (width 0.25) (layer B.Cu) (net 1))
 (segment (start 114 127.92) (end 114 125.38) (width 0.25) (layer B.Cu) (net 1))
 (segment (start 111 97.1038) (end 111 97.5) (width 0.4) (layer B.Cu) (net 1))
 (segment (start 111 82) (end 111 97.1038) (width 0.4) (layer B.Cu) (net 1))
 (segment (start 170.9456 78.1688) (end 160.0512 78.1688) (width 0.25) (layer B.Cu) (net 7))
 (segment (start 160.0512 78.1688) (end 157.54 80.68) (width 0.25) (layer B.Cu) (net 7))
 (segment (start 177.301 80.18) (end 177.301 79.3655) (width 0.25) (layer B.Cu) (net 7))
 (segment (start 177.301 79.3655) (end 176.1043 78.1688) (width 0.25) (layer B.Cu) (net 7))
 (segment (start 176.1043 78.1688) (end 170.9456 78.1688) (width 0.25) (layer B.Cu) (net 7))
 (segment (start 170.9456 78.1688) (end 170.9456 64.67) (width 0.25) (layer B.Cu) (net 7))
 (segment (start 170.9456 64.67) (end 175.32 64.67) (width 0.25) (layer B.Cu) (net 7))
 (segment (start 157.54 64.67) (end 170.9456 64.67) (width 0.25) (layer B.Cu) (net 7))
 (segment (start 175.32 94.3649) (end 173.9948 93.0397) (width 0.25) (layer B.Cu) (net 7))
 (segment (start 173.9948 93.0397) (end 173.9948 85.2122) (width 0.25) (layer B.Cu) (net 7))
 (segment (start 173.9948 85.2122) (end 177.301 81.906) (width 0.25) (layer B.Cu) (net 7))
 (segment (start 177.301 81.906) (end 177.301 80.18) (width 0.25) (layer B.Cu) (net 7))
 (segment (start 177.301 80.18) (end 191.7749 80.18) (width 0.25) (layer B.Cu) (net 7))
 (segment (start 193.1 80.18) (end 191.7749 80.18) (width 0.25) (layer B.Cu) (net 7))
 (segment (start 193.1 95.69) (end 191.7749 95.69) (width 0.25) (layer B.Cu) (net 7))
 (segment (start 175.32 95.0274) (end 191.1123 95.0274) (width 0.25) (layer B.Cu) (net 7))
 (segment (start 191.1123 95.0274) (end 191.7749 95.69) (width 0.25) (layer B.Cu) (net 7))
 (segment (start 175.32 95.0274) (end 175.32 94.3649) (width 0.25) (layer B.Cu) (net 7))
 (segment (start 175.32 95.69) (end 175.32 95.0274) (width 0.25) (layer B.Cu) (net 7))
 (segment (start 157.54 81.5051) (end 155.5199 83.5252) (width 0.25) (layer B.Cu) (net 7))
 (segment (start 155.5199 83.5252) (end 155.5199 92.3448) (width 0.25) (layer B.Cu) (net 7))
 (segment (start 155.5199 92.3448) (end 157.54 94.3649) (width 0.25) (layer B.Cu) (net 7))
 (segment (start 175.32 64.67) (end 193.1 64.67) (width 0.25) (layer B.Cu) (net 7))
 (segment (start 157.54 80.68) (end 157.54 81.5051) (width 0.25) (layer B.Cu) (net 7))
 (segment (start 157.54 80.18) (end 157.54 80.68) (width 0.25) (layer B.Cu) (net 7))
 (segment (start 157.54 95.69) (end 157.54 94.3649) (width 0.25) (layer B.Cu) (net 7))
 (segment (start 160.04 133) (end 162.2176 135.1776) (width 0.25) (layer B.Cu) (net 7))
 (segment (start 162.2176 135.1776) (end 174.5397 135.1776) (width 0.25) (layer B.Cu) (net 7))
 (segment (start 174.5397 135.1776) (end 176.0632 133.6541) (width 0.25) (layer B.Cu) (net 7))
 (segment (start 176.0632 133.6541) (end 176.0632 109.5127) (width 0.25) (layer B.Cu) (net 7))
 (segment (start 176.0632 109.5127) (end 173.9842 107.4337) (width 0.25) (layer B.Cu) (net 7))
 (segment (start 173.9842 107.4337) (end 173.9842 98.3509) (width 0.25) (layer B.Cu) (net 7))
 (segment (start 173.9842 98.3509) (end 175.32 97.0151) (width 0.25) (layer B.Cu) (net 7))
 (segment (start 175.32 95.69) (end 175.32 97.0151) (width 0.25) (layer B.Cu) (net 7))
 (segment (start 106.38 112.68) (end 104.3519 114.7081) (width 0.25) (layer B.Cu) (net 5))
 (segment (start 104.3519 114.7081) (end 104.3519 133.7875) (width 0.25) (layer B.Cu) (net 5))
 (segment (start 104.3519 133.7875) (end 106.2053 135.6409) (width 0.25) (layer B.Cu) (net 5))
 (segment (start 106.2053 135.6409) (end 130.1728 135.6409) (width 0.25) (layer B.Cu) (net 5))
 (segment (start 130.1728 135.6409) (end 131.1373 134.6764) (width 0.25) (layer B.Cu) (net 5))
 (segment (start 131.1373 134.6764) (end 131.1373 127.8627) (width 0.25) (layer B.Cu) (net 5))
 (segment (start 131.1373 127.8627) (end 132.5 126.5) (width 0.25) (layer B.Cu) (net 5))
 (segment (start 131.1373 134.6764) (end 154.346 134.6764) (width 0.25) (layer B.Cu) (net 5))
 (segment (start 154.346 134.6764) (end 156.0224 133) (width 0.25) (layer B.Cu) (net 5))
 (segment (start 157.5 133) (end 156.0224 133) (width 0.25) (layer B.Cu) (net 5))
 (segment (start 181.5 82.92) (end 181.5 88) (width 0.25) (layer B.Cu) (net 16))
 (segment (start 181.5 88) (end 180.0749 88) (width 0.25) (layer B.Cu) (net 16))
 (segment (start 180.0749 88) (end 177.7349 90.34) (width 0.25) (layer B.Cu) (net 16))
 (segment (start 177.7349 90.34) (end 175.32 90.34) (width 0.25) (layer B.Cu) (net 16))
 (segment (start 175.32 80.18) (end 175.32 81.5051) (width 0.25) (layer B.Cu) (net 15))
 (segment (start 172.04 133) (end 172.04 130.7269) (width 0.25) (layer B.Cu) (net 15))
 (segment (start 172.04 130.7269) (end 169.7345 128.4214) (width 0.25) (layer B.Cu) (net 15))
 (segment (start 169.7345 128.4214) (end 169.7345 87.0906) (width 0.25) (layer B.Cu) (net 15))
 (segment (start 169.7345 87.0906) (end 175.32 81.5051) (width 0.25) (layer B.Cu) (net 15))
 (segment (start 106.38 115.22) (end 105.002 116.598) (width 0.25) (layer B.Cu) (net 6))
 (segment (start 105.002 116.598) (end 105.002 133.5182) (width 0.25) (layer B.Cu) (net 6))
 (segment (start 105.002 133.5182) (end 106.4746 134.9908) (width 0.25) (layer B.Cu) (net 6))
 (segment (start 106.4746 134.9908) (end 121.5386 134.9908) (width 0.25) (layer B.Cu) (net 6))
 (segment (start 121.5386 134.9908) (end 131.3575 125.1719) (width 0.25) (layer B.Cu) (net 6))
 (segment (start 131.3575 125.1719) (end 133.0482 125.1719) (width 0.25) (layer B.Cu) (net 6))
 (segment (start 133.0482 125.1719) (end 133.8474 125.9711) (width 0.25) (layer B.Cu) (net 6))
 (segment (start 133.8474 125.9711) (end 133.8474 130.6526) (width 0.25) (layer B.Cu) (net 6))
 (segment (start 133.8474 130.6526) (end 132.5 132) (width 0.25) (layer B.Cu) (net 6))
 (segment (start 168.0224 133) (end 166.4883 131.4659) (width 0.25) (layer B.Cu) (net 6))
 (segment (start 166.4883 131.4659) (end 147.315 131.4659) (width 0.25) (layer B.Cu) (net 6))
 (segment (start 147.315 131.4659) (end 144.7799 134.001) (width 0.25) (layer B.Cu) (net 6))
 (segment (start 144.7799 134.001) (end 134.501 134.001) (width 0.25) (layer B.Cu) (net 6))
 (segment (start 134.501 134.001) (end 132.5 132) (width 0.25) (layer B.Cu) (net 6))
 (segment (start 169.5 133) (end 168.0224 133) (width 0.25) (layer B.Cu) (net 6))
 (segment (start 184.21 102.04) (end 179.13 102.04) (width 0.25) (layer B.Cu) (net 14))
 (segment (start 179.13 102.04) (end 175.32 105.85) (width 0.25) (layer B.Cu) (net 14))
 (segment (start 166.43 102.04) (end 167.9083 100.5617) (width 0.25) (layer B.Cu) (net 13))
 (segment (start 167.9083 100.5617) (end 167.9083 98.9468) (width 0.25) (layer B.Cu) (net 13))
 (segment (start 167.9083 98.9468) (end 167.0029 98.0414) (width 0.25) (layer B.Cu) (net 13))
 (segment (start 167.0029 98.0414) (end 165.3486 98.0414) (width 0.25) (layer B.Cu) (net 13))
 (segment (start 165.3486 98.0414) (end 157.54 105.85) (width 0.25) (layer B.Cu) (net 13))
 (segment (start 166.43 86.53) (end 161.35 86.53) (width 0.25) (layer B.Cu) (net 12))
 (segment (start 161.35 86.53) (end 157.54 90.34) (width 0.25) (layer B.Cu) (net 12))
 (segment (start 166.43 71.02) (end 161.35 71.02) (width 0.25) (layer B.Cu) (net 11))
 (segment (start 161.35 71.02) (end 157.54 74.83) (width 0.25) (layer B.Cu) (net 11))
 (segment (start 184.21 71.02) (end 179.13 71.02) (width 0.25) (layer B.Cu) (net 10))
 (segment (start 179.13 71.02) (end 175.32 74.83) (width 0.25) (layer B.Cu) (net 10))
 (segment (start 201.99 71.02) (end 196.91 71.02) (width 0.25) (layer B.Cu) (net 9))
 (segment (start 196.91 71.02) (end 193.1 74.83) (width 0.25) (layer B.Cu) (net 9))
 (segment (start 201.99 86.53) (end 196.91 86.53) (width 0.25) (layer B.Cu) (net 8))
 (segment (start 196.91 86.53) (end 193.1 90.34) (width 0.25) (layer B.Cu) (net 8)))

